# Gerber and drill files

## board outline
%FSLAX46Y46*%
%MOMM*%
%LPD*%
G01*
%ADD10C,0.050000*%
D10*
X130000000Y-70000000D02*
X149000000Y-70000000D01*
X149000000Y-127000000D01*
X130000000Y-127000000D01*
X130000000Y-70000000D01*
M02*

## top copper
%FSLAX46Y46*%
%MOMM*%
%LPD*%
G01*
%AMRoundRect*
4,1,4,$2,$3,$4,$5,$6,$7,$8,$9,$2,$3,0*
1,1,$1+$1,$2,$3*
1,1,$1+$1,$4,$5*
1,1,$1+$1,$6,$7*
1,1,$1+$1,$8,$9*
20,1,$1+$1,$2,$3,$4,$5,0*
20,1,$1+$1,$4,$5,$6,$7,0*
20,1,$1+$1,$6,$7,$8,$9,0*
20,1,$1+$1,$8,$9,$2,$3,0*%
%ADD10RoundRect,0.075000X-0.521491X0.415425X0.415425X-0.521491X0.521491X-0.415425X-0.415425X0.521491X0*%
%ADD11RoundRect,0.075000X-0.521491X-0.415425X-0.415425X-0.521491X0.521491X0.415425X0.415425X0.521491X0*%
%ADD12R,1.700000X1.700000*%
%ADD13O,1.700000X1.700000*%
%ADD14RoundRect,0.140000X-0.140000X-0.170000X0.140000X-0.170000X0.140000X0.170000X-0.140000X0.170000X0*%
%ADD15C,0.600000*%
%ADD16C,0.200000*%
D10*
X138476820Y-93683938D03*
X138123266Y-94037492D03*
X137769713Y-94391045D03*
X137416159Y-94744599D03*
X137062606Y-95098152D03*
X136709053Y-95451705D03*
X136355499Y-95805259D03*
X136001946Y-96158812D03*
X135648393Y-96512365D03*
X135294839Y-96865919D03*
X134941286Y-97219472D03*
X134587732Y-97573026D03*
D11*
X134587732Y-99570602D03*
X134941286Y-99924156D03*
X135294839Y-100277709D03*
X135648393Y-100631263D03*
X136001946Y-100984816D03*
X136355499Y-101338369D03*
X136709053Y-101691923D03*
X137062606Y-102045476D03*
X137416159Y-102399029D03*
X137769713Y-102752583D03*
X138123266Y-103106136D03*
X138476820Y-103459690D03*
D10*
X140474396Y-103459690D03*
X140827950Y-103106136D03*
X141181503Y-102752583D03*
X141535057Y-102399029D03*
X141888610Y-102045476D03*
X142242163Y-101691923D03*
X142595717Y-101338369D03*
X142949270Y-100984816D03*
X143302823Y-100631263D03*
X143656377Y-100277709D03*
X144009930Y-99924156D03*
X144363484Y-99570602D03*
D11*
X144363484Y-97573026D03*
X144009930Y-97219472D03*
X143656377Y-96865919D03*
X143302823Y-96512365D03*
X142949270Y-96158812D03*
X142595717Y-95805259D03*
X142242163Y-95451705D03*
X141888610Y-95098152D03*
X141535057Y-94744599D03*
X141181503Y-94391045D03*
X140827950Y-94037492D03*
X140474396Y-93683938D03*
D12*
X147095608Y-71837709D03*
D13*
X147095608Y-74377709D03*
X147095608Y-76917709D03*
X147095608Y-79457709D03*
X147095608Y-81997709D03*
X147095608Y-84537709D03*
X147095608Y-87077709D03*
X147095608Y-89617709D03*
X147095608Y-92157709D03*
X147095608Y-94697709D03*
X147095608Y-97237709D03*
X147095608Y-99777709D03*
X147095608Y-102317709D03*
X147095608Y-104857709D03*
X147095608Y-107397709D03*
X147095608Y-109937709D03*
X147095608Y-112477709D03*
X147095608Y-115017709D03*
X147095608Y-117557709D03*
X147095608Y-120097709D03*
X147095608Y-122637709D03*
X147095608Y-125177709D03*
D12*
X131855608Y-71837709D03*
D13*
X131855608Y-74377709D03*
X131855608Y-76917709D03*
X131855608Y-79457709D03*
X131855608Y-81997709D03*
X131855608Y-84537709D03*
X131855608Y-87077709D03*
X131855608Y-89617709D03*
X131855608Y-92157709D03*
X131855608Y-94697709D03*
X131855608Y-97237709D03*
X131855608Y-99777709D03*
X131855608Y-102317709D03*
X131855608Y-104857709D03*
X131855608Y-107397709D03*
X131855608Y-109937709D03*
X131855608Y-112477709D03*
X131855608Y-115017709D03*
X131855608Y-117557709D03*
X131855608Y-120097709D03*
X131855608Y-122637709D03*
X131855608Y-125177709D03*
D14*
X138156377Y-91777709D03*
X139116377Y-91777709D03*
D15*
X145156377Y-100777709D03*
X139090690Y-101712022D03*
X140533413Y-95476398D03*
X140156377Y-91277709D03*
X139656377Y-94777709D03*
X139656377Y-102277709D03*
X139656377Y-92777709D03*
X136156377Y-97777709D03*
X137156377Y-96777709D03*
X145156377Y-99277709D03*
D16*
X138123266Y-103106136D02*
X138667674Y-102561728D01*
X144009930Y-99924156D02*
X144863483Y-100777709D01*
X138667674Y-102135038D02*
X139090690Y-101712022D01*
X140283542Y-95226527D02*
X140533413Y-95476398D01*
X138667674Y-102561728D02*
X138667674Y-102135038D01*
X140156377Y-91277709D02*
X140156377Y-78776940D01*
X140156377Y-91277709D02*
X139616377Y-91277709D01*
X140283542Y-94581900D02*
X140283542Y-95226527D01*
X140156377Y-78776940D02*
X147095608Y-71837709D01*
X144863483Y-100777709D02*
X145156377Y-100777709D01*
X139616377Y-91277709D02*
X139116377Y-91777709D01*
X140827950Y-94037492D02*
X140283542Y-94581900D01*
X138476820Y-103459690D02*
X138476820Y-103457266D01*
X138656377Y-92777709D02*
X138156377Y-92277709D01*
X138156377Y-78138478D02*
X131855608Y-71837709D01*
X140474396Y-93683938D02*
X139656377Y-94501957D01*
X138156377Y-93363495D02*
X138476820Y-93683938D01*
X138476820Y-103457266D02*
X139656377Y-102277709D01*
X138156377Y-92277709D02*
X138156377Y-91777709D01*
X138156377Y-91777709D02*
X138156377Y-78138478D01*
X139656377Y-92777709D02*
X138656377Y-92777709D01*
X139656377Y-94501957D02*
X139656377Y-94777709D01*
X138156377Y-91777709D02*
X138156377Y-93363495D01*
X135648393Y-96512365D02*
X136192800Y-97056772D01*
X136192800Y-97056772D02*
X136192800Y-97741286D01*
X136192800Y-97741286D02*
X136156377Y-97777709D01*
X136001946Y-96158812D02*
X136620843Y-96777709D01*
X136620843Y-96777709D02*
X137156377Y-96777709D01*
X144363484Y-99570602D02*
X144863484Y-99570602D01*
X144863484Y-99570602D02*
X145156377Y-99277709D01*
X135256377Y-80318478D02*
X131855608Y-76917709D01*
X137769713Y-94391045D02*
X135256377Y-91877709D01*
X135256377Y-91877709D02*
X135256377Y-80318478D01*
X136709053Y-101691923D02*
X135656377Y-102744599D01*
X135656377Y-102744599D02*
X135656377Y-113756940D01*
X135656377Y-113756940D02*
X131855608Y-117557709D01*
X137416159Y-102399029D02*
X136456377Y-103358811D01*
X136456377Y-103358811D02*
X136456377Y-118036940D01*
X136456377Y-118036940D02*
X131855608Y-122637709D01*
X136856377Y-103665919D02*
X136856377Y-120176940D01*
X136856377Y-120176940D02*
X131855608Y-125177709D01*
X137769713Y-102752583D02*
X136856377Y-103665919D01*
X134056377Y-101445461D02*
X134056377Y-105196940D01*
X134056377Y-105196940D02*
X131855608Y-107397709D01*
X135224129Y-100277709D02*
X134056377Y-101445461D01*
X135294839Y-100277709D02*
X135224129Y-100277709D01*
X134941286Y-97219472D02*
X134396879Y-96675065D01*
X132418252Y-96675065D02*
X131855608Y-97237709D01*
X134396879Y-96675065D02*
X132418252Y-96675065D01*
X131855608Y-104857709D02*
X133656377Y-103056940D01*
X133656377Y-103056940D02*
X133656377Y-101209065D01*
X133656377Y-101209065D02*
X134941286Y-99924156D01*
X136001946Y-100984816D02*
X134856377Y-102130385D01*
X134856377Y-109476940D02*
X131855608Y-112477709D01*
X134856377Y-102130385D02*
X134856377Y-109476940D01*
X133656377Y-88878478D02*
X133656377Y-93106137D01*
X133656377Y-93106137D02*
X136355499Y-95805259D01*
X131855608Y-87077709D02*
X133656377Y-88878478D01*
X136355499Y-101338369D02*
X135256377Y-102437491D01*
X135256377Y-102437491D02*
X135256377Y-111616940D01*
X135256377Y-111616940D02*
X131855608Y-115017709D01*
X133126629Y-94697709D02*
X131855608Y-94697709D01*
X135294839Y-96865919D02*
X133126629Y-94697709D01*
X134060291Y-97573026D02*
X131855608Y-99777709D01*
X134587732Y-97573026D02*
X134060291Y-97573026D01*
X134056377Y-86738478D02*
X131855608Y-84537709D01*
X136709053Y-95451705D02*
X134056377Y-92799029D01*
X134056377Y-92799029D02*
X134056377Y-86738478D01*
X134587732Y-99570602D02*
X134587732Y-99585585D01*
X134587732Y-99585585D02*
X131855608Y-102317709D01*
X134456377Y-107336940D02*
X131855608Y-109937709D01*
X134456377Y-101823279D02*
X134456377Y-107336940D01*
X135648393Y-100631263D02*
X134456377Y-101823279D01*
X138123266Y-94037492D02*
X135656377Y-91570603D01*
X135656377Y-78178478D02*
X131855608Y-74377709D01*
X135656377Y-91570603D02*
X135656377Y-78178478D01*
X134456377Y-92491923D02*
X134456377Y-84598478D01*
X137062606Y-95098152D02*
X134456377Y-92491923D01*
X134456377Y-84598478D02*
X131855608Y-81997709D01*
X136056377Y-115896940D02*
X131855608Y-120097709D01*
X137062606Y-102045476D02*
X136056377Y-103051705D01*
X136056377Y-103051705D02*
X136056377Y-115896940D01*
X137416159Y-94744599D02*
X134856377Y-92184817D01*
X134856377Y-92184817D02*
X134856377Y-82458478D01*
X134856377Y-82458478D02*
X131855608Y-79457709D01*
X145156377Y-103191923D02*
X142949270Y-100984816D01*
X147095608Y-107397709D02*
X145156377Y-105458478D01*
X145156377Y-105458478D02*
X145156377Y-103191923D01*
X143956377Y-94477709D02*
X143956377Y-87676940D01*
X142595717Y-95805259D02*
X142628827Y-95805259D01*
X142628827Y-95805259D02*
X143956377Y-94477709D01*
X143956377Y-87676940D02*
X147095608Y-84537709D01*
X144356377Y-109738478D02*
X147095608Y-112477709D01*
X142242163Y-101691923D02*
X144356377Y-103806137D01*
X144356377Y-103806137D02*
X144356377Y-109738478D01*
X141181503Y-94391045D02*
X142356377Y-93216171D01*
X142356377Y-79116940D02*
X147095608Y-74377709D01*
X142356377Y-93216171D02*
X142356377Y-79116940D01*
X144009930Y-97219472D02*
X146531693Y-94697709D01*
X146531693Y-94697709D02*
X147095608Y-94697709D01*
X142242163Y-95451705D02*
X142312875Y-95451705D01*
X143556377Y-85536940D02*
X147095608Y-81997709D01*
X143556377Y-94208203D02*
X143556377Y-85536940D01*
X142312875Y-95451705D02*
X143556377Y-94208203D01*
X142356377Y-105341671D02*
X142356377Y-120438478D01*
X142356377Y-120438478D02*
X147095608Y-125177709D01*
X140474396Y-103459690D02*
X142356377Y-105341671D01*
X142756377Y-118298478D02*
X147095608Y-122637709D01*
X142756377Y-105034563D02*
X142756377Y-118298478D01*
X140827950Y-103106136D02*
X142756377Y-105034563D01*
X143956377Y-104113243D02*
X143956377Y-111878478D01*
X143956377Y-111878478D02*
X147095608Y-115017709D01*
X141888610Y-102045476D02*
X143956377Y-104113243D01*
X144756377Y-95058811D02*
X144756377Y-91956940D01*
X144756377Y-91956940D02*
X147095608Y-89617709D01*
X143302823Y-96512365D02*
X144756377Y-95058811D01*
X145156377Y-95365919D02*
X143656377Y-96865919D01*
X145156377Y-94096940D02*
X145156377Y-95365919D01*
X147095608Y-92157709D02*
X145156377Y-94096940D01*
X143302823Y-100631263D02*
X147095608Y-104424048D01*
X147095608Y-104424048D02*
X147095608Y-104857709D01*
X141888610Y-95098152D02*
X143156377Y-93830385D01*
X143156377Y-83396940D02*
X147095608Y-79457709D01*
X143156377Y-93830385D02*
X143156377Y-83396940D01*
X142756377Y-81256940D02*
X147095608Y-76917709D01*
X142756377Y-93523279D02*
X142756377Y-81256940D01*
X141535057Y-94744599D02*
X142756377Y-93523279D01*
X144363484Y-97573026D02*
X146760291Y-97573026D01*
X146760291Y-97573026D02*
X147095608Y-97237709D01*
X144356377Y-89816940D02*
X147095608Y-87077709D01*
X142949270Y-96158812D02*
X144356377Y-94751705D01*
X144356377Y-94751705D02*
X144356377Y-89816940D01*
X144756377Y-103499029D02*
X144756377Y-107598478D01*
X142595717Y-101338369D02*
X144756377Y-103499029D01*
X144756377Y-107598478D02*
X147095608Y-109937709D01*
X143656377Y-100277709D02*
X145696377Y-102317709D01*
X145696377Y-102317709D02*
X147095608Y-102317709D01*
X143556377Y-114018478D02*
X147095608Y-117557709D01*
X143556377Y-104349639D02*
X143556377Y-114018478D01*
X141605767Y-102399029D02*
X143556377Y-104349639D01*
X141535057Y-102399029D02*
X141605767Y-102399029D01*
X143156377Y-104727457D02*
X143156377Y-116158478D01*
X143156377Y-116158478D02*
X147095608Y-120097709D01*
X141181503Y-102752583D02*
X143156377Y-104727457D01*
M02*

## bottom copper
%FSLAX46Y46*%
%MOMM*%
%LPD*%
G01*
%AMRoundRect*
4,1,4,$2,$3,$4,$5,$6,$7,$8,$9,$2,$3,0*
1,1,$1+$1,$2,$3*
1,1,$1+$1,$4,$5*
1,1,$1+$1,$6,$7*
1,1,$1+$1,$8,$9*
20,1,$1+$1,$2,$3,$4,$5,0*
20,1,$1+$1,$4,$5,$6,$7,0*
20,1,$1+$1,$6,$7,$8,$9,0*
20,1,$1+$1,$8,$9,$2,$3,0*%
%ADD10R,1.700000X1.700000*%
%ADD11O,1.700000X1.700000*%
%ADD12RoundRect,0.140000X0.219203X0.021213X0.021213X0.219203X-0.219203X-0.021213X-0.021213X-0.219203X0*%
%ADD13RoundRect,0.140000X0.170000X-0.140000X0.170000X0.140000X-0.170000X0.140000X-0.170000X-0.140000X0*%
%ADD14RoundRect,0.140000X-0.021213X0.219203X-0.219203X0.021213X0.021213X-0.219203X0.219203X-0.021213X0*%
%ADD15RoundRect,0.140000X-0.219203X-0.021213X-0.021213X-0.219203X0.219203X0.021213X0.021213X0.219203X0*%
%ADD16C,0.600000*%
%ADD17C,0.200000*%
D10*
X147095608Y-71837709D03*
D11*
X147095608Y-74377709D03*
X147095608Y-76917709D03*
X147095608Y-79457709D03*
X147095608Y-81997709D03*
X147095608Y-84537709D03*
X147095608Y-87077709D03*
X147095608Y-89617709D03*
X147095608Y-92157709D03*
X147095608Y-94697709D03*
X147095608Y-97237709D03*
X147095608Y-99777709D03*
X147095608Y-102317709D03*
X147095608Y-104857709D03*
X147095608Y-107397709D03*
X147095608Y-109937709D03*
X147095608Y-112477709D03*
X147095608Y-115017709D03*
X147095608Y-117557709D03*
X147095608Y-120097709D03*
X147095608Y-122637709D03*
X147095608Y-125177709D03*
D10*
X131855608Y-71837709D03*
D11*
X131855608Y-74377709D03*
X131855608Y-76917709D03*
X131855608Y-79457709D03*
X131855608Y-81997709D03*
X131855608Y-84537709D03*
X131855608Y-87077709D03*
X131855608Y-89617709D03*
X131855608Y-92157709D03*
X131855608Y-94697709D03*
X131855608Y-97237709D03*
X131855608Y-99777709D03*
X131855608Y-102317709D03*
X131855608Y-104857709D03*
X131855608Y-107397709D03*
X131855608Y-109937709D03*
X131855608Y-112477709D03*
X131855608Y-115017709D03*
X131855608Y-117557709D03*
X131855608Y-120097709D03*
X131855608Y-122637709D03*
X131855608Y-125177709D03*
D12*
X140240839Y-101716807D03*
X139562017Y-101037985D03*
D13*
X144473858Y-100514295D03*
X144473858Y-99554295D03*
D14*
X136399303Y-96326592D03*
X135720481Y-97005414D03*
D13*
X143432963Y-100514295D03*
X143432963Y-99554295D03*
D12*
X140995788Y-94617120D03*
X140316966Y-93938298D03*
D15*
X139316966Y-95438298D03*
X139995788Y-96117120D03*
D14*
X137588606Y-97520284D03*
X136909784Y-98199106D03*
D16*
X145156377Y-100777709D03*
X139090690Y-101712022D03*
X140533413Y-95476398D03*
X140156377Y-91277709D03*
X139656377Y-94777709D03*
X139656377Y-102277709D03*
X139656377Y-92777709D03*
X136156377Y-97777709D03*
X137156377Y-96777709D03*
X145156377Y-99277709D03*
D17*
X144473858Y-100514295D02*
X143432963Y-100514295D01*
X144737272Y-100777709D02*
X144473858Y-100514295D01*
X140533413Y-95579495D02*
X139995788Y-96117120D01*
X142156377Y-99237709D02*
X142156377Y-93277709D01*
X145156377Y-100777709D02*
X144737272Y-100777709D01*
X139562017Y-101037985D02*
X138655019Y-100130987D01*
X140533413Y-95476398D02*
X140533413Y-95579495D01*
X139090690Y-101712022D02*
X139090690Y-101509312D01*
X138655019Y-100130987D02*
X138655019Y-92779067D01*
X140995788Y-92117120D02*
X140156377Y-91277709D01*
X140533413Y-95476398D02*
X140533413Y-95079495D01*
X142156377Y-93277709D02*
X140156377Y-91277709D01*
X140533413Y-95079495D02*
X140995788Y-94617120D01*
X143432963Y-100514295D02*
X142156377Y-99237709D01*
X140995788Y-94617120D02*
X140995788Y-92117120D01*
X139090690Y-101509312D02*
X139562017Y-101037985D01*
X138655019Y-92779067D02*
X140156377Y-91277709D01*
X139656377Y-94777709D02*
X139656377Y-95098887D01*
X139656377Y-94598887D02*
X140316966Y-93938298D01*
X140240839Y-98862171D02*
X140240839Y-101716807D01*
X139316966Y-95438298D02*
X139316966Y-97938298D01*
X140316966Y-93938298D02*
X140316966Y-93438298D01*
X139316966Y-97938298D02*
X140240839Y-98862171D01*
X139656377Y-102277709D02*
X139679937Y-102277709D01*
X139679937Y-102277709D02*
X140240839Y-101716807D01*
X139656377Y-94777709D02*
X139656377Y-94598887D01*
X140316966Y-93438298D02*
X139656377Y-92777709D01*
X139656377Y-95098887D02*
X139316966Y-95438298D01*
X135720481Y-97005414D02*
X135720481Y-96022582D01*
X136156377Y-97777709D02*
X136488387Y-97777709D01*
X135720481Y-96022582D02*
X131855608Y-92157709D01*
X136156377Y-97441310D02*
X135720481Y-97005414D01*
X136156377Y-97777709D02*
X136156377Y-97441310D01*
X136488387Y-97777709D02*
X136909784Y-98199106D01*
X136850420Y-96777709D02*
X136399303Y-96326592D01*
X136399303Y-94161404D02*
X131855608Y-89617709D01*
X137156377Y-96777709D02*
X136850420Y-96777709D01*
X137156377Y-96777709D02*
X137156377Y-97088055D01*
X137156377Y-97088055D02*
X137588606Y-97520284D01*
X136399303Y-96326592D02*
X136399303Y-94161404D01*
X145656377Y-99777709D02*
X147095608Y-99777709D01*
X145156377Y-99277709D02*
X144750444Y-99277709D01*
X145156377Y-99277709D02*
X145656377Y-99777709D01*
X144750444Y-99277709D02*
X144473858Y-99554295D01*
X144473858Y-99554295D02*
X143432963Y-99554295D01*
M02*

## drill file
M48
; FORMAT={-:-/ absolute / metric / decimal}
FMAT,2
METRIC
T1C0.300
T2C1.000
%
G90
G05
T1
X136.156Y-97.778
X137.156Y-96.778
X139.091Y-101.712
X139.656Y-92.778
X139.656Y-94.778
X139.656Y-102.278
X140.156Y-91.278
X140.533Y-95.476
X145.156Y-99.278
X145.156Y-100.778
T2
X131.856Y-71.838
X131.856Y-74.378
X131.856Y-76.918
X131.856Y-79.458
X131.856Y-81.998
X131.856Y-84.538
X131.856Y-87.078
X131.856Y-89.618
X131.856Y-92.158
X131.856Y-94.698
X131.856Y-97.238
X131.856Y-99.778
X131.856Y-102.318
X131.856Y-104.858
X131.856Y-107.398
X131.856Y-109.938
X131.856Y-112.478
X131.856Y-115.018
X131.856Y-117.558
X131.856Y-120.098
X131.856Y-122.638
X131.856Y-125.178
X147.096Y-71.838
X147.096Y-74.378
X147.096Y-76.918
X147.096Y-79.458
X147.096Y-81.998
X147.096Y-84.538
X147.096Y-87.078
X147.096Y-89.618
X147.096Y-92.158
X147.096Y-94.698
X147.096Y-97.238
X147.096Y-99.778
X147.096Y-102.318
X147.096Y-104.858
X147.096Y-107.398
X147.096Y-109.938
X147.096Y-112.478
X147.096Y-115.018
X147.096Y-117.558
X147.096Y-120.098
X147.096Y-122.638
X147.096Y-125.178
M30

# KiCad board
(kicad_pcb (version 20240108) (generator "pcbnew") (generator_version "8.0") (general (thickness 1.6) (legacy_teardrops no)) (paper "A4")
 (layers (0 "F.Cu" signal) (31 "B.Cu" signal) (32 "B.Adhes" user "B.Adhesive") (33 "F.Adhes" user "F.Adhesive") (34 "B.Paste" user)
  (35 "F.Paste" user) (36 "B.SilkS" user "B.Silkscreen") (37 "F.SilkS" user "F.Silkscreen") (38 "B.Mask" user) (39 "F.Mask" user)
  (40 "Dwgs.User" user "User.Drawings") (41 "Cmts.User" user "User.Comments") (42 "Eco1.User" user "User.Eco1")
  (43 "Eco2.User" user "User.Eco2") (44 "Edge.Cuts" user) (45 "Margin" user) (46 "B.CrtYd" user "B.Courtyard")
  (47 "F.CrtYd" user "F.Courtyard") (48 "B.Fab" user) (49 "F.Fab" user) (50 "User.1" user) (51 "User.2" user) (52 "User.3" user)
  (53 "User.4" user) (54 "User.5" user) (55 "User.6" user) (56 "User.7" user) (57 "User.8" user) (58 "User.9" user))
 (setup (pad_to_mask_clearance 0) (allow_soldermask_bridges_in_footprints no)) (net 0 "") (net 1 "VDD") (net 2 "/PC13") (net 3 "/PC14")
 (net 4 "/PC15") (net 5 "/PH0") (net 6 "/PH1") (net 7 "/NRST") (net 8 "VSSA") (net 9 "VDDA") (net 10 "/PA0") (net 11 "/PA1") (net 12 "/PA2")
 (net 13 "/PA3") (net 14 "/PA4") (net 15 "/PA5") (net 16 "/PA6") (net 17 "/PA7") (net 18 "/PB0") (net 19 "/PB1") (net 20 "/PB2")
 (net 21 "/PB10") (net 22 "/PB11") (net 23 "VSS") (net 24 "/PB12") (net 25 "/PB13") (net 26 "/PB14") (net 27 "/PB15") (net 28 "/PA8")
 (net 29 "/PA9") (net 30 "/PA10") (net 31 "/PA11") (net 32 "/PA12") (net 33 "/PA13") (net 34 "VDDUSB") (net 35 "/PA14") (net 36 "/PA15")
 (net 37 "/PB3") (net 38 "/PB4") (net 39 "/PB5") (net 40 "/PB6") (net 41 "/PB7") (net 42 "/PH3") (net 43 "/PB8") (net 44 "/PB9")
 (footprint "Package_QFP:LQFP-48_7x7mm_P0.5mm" (layer "F.Cu") (at 139.475608 98.571814 -45)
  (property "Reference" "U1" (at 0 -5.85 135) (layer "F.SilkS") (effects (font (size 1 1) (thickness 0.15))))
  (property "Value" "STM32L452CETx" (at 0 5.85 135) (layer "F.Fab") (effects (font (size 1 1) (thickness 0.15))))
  (pad "1" smd roundrect (at -4.1625 -2.75 315) (size 1.475 0.3) (layers "F.Cu" "F.Paste" "F.Mask") (roundrect_rratio 0.25) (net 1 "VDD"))
  (pad "2" smd roundrect (at -4.1625 -2.25 315) (size 1.475 0.3) (layers "F.Cu" "F.Paste" "F.Mask") (roundrect_rratio 0.25) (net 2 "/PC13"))
  (pad "3" smd roundrect (at -4.1625 -1.75 315) (size 1.475 0.3) (layers "F.Cu" "F.Paste" "F.Mask") (roundrect_rratio 0.25) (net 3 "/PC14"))
  (pad "4" smd roundrect (at -4.1625 -1.249999 315) (size 1.475 0.3) (layers "F.Cu" "F.Paste" "F.Mask") (roundrect_rratio 0.25)
   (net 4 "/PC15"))
  (pad "5" smd roundrect (at -4.1625 -0.75 315) (size 1.475 0.3) (layers "F.Cu" "F.Paste" "F.Mask") (roundrect_rratio 0.25) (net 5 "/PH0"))
  (pad "6" smd roundrect (at -4.1625 -0.25 315) (size 1.475 0.3) (layers "F.Cu" "F.Paste" "F.Mask") (roundrect_rratio 0.25) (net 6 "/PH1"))
  (pad "7" smd roundrect (at -4.1625 0.25 315) (size 1.475 0.3) (layers "F.Cu" "F.Paste" "F.Mask") (roundrect_rratio 0.25) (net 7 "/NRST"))
  (pad "8" smd roundrect (at -4.1625 0.75 315) (size 1.475 0.3) (layers "F.Cu" "F.Paste" "F.Mask") (roundrect_rratio 0.25) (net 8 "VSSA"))
  (pad "9" smd roundrect (at -4.1625 1.249999 315) (size 1.475 0.3) (layers "F.Cu" "F.Paste" "F.Mask") (roundrect_rratio 0.25)
   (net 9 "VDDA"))
  (pad "10" smd roundrect (at -4.1625 1.75 315) (size 1.475 0.3) (layers "F.Cu" "F.Paste" "F.Mask") (roundrect_rratio 0.25) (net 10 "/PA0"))
  (pad "11" smd roundrect (at -4.1625 2.25 315) (size 1.475 0.3) (layers "F.Cu" "F.Paste" "F.Mask") (roundrect_rratio 0.25) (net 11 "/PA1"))
  (pad "12" smd roundrect (at -4.1625 2.75 315) (size 1.475 0.3) (layers "F.Cu" "F.Paste" "F.Mask") (roundrect_rratio 0.25) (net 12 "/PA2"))
  (pad "13" smd roundrect (at -2.75 4.1625 315) (size 0.3 1.475) (layers "F.Cu" "F.Paste" "F.Mask") (roundrect_rratio 0.25) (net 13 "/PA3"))
  (pad "14" smd roundrect (at -2.25 4.1625 315) (size 0.3 1.475) (layers "F.Cu" "F.Paste" "F.Mask") (roundrect_rratio 0.25) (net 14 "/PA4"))
  (pad "15" smd roundrect (at -1.75 4.1625 315) (size 0.3 1.475) (layers "F.Cu" "F.Paste" "F.Mask") (roundrect_rratio 0.25) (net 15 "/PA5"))
  (pad "16" smd roundrect (at -1.249999 4.1625 315) (size 0.3 1.475) (layers "F.Cu" "F.Paste" "F.Mask") (roundrect_rratio 0.25)
   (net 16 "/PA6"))
  (pad "17" smd roundrect (at -0.75 4.1625 315) (size 0.3 1.475) (layers "F.Cu" "F.Paste" "F.Mask") (roundrect_rratio 0.25) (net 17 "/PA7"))
  (pad "18" smd roundrect (at -0.25 4.1625 315) (size 0.3 1.475) (layers "F.Cu" "F.Paste" "F.Mask") (roundrect_rratio 0.25) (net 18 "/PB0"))
  (pad "19" smd roundrect (at 0.25 4.1625 315) (size 0.3 1.475) (layers "F.Cu" "F.Paste" "F.Mask") (roundrect_rratio 0.25) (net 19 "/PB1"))
  (pad "20" smd roundrect (at 0.75 4.1625 315) (size 0.3 1.475) (layers "F.Cu" "F.Paste" "F.Mask") (roundrect_rratio 0.25) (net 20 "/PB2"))
  (pad "21" smd roundrect (at 1.249999 4.1625 315) (size 0.3 1.475) (layers "F.Cu" "F.Paste" "F.Mask") (roundrect_rratio 0.25)
   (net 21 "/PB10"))
  (pad "22" smd roundrect (at 1.75 4.1625 315) (size 0.3 1.475) (layers "F.Cu" "F.Paste" "F.Mask") (roundrect_rratio 0.25) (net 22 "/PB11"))
  (pad "23" smd roundrect (at 2.25 4.1625 315) (size 0.3 1.475) (layers "F.Cu" "F.Paste" "F.Mask") (roundrect_rratio 0.25) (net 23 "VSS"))
  (pad "24" smd roundrect (at 2.75 4.1625 315) (size 0.3 1.475) (layers "F.Cu" "F.Paste" "F.Mask") (roundrect_rratio 0.25) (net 1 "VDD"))
  (pad "25" smd roundrect (at 4.1625 2.75 315) (size 1.475 0.3) (layers "F.Cu" "F.Paste" "F.Mask") (roundrect_rratio 0.25) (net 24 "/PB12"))
  (pad "26" smd roundrect (at 4.1625 2.25 315) (size 1.475 0.3) (layers "F.Cu" "F.Paste" "F.Mask") (roundrect_rratio 0.25) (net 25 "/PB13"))
  (pad "27" smd roundrect (at 4.1625 1.75 315) (size 1.475 0.3) (layers "F.Cu" "F.Paste" "F.Mask") (roundrect_rratio 0.25) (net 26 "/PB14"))
  (pad "28" smd roundrect (at 4.1625 1.249999 315) (size 1.475 0.3) (layers "F.Cu" "F.Paste" "F.Mask") (roundrect_rratio 0.25)
   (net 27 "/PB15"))
  (pad "29" smd roundrect (at 4.1625 0.75 315) (size 1.475 0.3) (layers "F.Cu" "F.Paste" "F.Mask") (roundrect_rratio 0.25) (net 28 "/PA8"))
  (pad "30" smd roundrect (at 4.1625 0.25 315) (size 1.475 0.3) (layers "F.Cu" "F.Paste" "F.Mask") (roundrect_rratio 0.25) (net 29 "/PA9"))
  (pad "31" smd roundrect (at 4.1625 -0.25 315) (size 1.475 0.3) (layers "F.Cu" "F.Paste" "F.Mask") (roundrect_rratio 0.25) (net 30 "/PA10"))
  (pad "32" smd roundrect (at 4.1625 -0.75 315) (size 1.475 0.3) (layers "F.Cu" "F.Paste" "F.Mask") (roundrect_rratio 0.25) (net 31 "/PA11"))
  (pad "33" smd roundrect (at 4.1625 -1.249999 315) (size 1.475 0.3) (layers "F.Cu" "F.Paste" "F.Mask") (roundrect_rratio 0.25)
   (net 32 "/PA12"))
  (pad "34" smd roundrect (at 4.1625 -1.75 315) (size 1.475 0.3) (layers "F.Cu" "F.Paste" "F.Mask") (roundrect_rratio 0.25) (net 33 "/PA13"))
  (pad "35" smd roundrect (at 4.1625 -2.25 315) (size 1.475 0.3) (layers "F.Cu" "F.Paste" "F.Mask") (roundrect_rratio 0.25) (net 23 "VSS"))
  (pad "36" smd roundrect (at 4.1625 -2.75 315) (size 1.475 0.3) (layers "F.Cu" "F.Paste" "F.Mask") (roundrect_rratio 0.25)
   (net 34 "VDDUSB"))
  (pad "37" smd roundrect (at 2.75 -4.1625 315) (size 0.3 1.475) (layers "F.Cu" "F.Paste" "F.Mask") (roundrect_rratio 0.25) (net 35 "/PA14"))
  (pad "38" smd roundrect (at 2.25 -4.1625 315) (size 0.3 1.475) (layers "F.Cu" "F.Paste" "F.Mask") (roundrect_rratio 0.25) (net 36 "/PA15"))
  (pad "39" smd roundrect (at 1.75 -4.1625 315) (size 0.3 1.475) (layers "F.Cu" "F.Paste" "F.Mask") (roundrect_rratio 0.25) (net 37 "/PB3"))
  (pad "40" smd roundrect (at 1.249999 -4.1625 315) (size 0.3 1.475) (layers "F.Cu" "F.Paste" "F.Mask") (roundrect_rratio 0.25)
   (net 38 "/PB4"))
  (pad "41" smd roundrect (at 0.75 -4.1625 315) (size 0.3 1.475) (layers "F.Cu" "F.Paste" "F.Mask") (roundrect_rratio 0.25) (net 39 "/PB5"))
  (pad "42" smd roundrect (at 0.25 -4.1625 315) (size 0.3 1.475) (layers "F.Cu" "F.Paste" "F.Mask") (roundrect_rratio 0.25) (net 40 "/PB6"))
  (pad "43" smd roundrect (at -0.25 -4.1625 315) (size 0.3 1.475) (layers "F.Cu" "F.Paste" "F.Mask") (roundrect_rratio 0.25) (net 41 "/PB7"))
  (pad "44" smd roundrect (at -0.75 -4.1625 315) (size 0.3 1.475) (layers "F.Cu" "F.Paste" "F.Mask") (roundrect_rratio 0.25) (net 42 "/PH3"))
  (pad "45" smd roundrect (at -1.249999 -4.1625 315) (size 0.3 1.475) (layers "F.Cu" "F.Paste" "F.Mask") (roundrect_rratio 0.25)
   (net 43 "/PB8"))
  (pad "46" smd roundrect (at -1.75 -4.1625 315) (size 0.3 1.475) (layers "F.Cu" "F.Paste" "F.Mask") (roundrect_rratio 0.25) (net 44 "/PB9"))
  (pad "47" smd roundrect (at -2.25 -4.1625 315) (size 0.3 1.475) (layers "F.Cu" "F.Paste" "F.Mask") (roundrect_rratio 0.25) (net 23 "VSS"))
  (pad "48" smd roundrect (at -2.75 -4.1625 315) (size 0.3 1.475) (layers "F.Cu" "F.Paste" "F.Mask") (roundrect_rratio 0.25) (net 1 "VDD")))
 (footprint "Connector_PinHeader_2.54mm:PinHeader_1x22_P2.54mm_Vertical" (layer "F.Cu") (at 147.095608 71.837709)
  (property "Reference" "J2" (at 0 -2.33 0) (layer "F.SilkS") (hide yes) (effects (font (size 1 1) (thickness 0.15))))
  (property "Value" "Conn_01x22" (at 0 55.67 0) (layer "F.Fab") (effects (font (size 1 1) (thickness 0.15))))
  (pad "1" thru_hole rect (at 0 0) (size 1.7 1.7) (drill 1) (layers "*.Cu" "*.Mask") (remove_unused_layers no) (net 23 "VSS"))
  (pad "2" thru_hole oval (at 0 2.54) (size 1.7 1.7) (drill 1) (layers "*.Cu" "*.Mask") (remove_unused_layers no) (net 44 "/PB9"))
  (pad "3" thru_hole oval (at 0 5.08) (size 1.7 1.7) (drill 1) (layers "*.Cu" "*.Mask") (remove_unused_layers no) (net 43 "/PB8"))
  (pad "4" thru_hole oval (at 0 7.62) (size 1.7 1.7) (drill 1) (layers "*.Cu" "*.Mask") (remove_unused_layers no) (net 42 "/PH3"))
  (pad "5" thru_hole oval (at 0 10.16) (size 1.7 1.7) (drill 1) (layers "*.Cu" "*.Mask") (remove_unused_layers no) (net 41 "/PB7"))
  (pad "6" thru_hole oval (at 0 12.7) (size 1.7 1.7) (drill 1) (layers "*.Cu" "*.Mask") (remove_unused_layers no) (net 40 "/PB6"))
  (pad "7" thru_hole oval (at 0 15.24) (size 1.7 1.7) (drill 1) (layers "*.Cu" "*.Mask") (remove_unused_layers no) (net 39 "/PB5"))
  (pad "8" thru_hole oval (at 0 17.78) (size 1.7 1.7) (drill 1) (layers "*.Cu" "*.Mask") (remove_unused_layers no) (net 38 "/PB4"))
  (pad "9" thru_hole oval (at 0 20.32) (size 1.7 1.7) (drill 1) (layers "*.Cu" "*.Mask") (remove_unused_layers no) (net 37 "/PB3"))
  (pad "10" thru_hole oval (at 0 22.86) (size 1.7 1.7) (drill 1) (layers "*.Cu" "*.Mask") (remove_unused_layers no) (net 36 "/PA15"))
  (pad "11" thru_hole oval (at 0 25.4) (size 1.7 1.7) (drill 1) (layers "*.Cu" "*.Mask") (remove_unused_layers no) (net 35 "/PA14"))
  (pad "12" thru_hole oval (at 0 27.94) (size 1.7 1.7) (drill 1) (layers "*.Cu" "*.Mask") (remove_unused_layers no) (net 34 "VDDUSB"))
  (pad "13" thru_hole oval (at 0 30.48) (size 1.7 1.7) (drill 1) (layers "*.Cu" "*.Mask") (remove_unused_layers no) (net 33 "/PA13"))
  (pad "14" thru_hole oval (at 0 33.02) (size 1.7 1.7) (drill 1) (layers "*.Cu" "*.Mask") (remove_unused_layers no) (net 32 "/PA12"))
  (pad "15" thru_hole oval (at 0 35.56) (size 1.7 1.7) (drill 1) (layers "*.Cu" "*.Mask") (remove_unused_layers no) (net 31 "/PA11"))
  (pad "16" thru_hole oval (at 0 38.1) (size 1.7 1.7) (drill 1) (layers "*.Cu" "*.Mask") (remove_unused_layers no) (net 30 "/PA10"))
  (pad "17" thru_hole oval (at 0 40.64) (size 1.7 1.7) (drill 1) (layers "*.Cu" "*.Mask") (remove_unused_layers no) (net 29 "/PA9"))
  (pad "18" thru_hole oval (at 0 43.18) (size 1.7 1.7) (drill 1) (layers "*.Cu" "*.Mask") (remove_unused_layers no) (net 28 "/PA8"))
  (pad "19" thru_hole oval (at 0 45.72) (size 1.7 1.7) (drill 1) (layers "*.Cu" "*.Mask") (remove_unused_layers no) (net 27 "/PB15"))
  (pad "20" thru_hole oval (at 0 48.26) (size 1.7 1.7) (drill 1) (layers "*.Cu" "*.Mask") (remove_unused_layers no) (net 26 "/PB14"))
  (pad "21" thru_hole oval (at 0 50.8) (size 1.7 1.7) (drill 1) (layers "*.Cu" "*.Mask") (remove_unused_layers no) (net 25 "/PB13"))
  (pad "22" thru_hole oval (at 0 53.34) (size 1.7 1.7) (drill 1) (layers "*.Cu" "*.Mask") (remove_unused_layers no) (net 24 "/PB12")))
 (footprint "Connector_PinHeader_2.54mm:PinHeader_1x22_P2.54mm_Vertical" (layer "F.Cu") (at 131.855608 71.837709)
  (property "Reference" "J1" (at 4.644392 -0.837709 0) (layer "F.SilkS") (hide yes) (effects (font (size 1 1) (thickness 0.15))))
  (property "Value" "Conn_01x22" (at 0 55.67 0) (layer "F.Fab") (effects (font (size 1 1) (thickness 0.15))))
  (pad "1" thru_hole rect (at 0 0) (size 1.7 1.7) (drill 1) (layers "*.Cu" "*.Mask") (remove_unused_layers no) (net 1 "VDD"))
  (pad "2" thru_hole oval (at 0 2.54) (size 1.7 1.7) (drill 1) (layers "*.Cu" "*.Mask") (remove_unused_layers no) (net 2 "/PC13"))
  (pad "3" thru_hole oval (at 0 5.08) (size 1.7 1.7) (drill 1) (layers "*.Cu" "*.Mask") (remove_unused_layers no) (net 3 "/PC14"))
  (pad "4" thru_hole oval (at 0 7.62) (size 1.7 1.7) (drill 1) (layers "*.Cu" "*.Mask") (remove_unused_layers no) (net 4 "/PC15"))
  (pad "5" thru_hole oval (at 0 10.16) (size 1.7 1.7) (drill 1) (layers "*.Cu" "*.Mask") (remove_unused_layers no) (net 5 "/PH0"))
  (pad "6" thru_hole oval (at 0 12.7) (size 1.7 1.7) (drill 1) (layers "*.Cu" "*.Mask") (remove_unused_layers no) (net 6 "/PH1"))
  (pad "7" thru_hole oval (at 0 15.24) (size 1.7 1.7) (drill 1) (layers "*.Cu" "*.Mask") (remove_unused_layers no) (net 7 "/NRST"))
  (pad "8" thru_hole oval (at 0 17.78) (size 1.7 1.7) (drill 1) (layers "*.Cu" "*.Mask") (remove_unused_layers no) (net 8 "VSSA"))
  (pad "9" thru_hole oval (at 0 20.32) (size 1.7 1.7) (drill 1) (layers "*.Cu" "*.Mask") (remove_unused_layers no) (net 9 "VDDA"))
  (pad "10" thru_hole oval (at 0 22.86) (size 1.7 1.7) (drill 1) (layers "*.Cu" "*.Mask") (remove_unused_layers no) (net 10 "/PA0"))
  (pad "11" thru_hole oval (at 0 25.4) (size 1.7 1.7) (drill 1) (layers "*.Cu" "*.Mask") (remove_unused_layers no) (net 11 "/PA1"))
  (pad "12" thru_hole oval (at 0 27.94) (size 1.7 1.7) (drill 1) (layers "*.Cu" "*.Mask") (remove_unused_layers no) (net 12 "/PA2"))
  (pad "13" thru_hole oval (at 0 30.48) (size 1.7 1.7) (drill 1) (layers "*.Cu" "*.Mask") (remove_unused_layers no) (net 13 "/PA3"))
  (pad "14" thru_hole oval (at 0 33.02) (size 1.7 1.7) (drill 1) (layers "*.Cu" "*.Mask") (remove_unused_layers no) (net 14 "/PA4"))
  (pad "15" thru_hole oval (at 0 35.56) (size 1.7 1.7) (drill 1) (layers "*.Cu" "*.Mask") (remove_unused_layers no) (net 15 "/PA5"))
  (pad "16" thru_hole oval (at 0 38.1) (size 1.7 1.7) (drill 1) (layers "*.Cu" "*.Mask") (remove_unused_layers no) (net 16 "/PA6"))
  (pad "17" thru_hole oval (at 0 40.64) (size 1.7 1.7) (drill 1) (layers "*.Cu" "*.Mask") (remove_unused_layers no) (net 17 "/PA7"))
  (pad "18" thru_hole oval (at 0 43.18) (size 1.7 1.7) (drill 1) (layers "*.Cu" "*.Mask") (remove_unused_layers no) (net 18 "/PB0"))
  (pad "19" thru_hole oval (at 0 45.72) (size 1.7 1.7) (drill 1) (layers "*.Cu" "*.Mask") (remove_unused_layers no) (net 19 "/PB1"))
  (pad "20" thru_hole oval (at 0 48.26) (size 1.7 1.7) (drill 1) (layers "*.Cu" "*.Mask") (remove_unused_layers no) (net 20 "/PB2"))
  (pad "21" thru_hole oval (at 0 50.8) (size 1.7 1.7) (drill 1) (layers "*.Cu" "*.Mask") (remove_unused_layers no) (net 21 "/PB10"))
  (pad "22" thru_hole oval (at 0 53.34) (size 1.7 1.7) (drill 1) (layers "*.Cu" "*.Mask") (remove_unused_layers no) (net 22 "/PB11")))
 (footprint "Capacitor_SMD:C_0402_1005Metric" (layer "F.Cu") (at 138.636377 91.777709)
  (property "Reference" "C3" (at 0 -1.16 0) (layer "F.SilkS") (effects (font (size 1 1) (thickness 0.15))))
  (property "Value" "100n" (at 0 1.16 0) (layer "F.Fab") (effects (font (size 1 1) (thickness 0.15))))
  (pad "1" smd roundrect (at -0.48 0) (size 0.56 0.62) (layers "F.Cu" "F.Paste" "F.Mask") (roundrect_rratio 0.25) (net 1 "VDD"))
  (pad "2" smd roundrect (at 0.48 0) (size 0.56 0.62) (layers "F.Cu" "F.Paste" "F.Mask") (roundrect_rratio 0.25) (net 23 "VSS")))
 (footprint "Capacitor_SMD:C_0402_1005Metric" (layer "B.Cu") (at 139.901428 101.377396 135)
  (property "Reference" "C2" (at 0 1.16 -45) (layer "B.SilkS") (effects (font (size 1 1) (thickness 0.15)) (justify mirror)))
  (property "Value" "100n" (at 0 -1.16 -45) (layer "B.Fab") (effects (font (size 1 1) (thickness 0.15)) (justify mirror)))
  (pad "1" smd roundrect (at -0.48 0 135) (size 0.56 0.62) (layers "B.Cu" "B.Paste" "B.Mask") (roundrect_rratio 0.25) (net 1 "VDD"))
  (pad "2" smd roundrect (at 0.48 0 135) (size 0.56 0.62) (layers "B.Cu" "B.Paste" "B.Mask") (roundrect_rratio 0.25) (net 23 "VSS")))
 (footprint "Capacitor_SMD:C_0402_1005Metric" (layer "B.Cu") (at 144.473858 100.034295 90)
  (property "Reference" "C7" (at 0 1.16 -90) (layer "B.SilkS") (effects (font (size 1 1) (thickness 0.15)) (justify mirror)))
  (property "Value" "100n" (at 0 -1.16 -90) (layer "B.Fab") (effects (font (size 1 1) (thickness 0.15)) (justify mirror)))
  (pad "1" smd roundrect (at -0.48 0 90) (size 0.56 0.62) (layers "B.Cu" "B.Paste" "B.Mask") (roundrect_rratio 0.25) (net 23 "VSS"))
  (pad "2" smd roundrect (at 0.48 0 90) (size 0.56 0.62) (layers "B.Cu" "B.Paste" "B.Mask") (roundrect_rratio 0.25) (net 34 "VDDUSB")))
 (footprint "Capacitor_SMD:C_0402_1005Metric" (layer "B.Cu") (at 136.059892 96.666003 -135)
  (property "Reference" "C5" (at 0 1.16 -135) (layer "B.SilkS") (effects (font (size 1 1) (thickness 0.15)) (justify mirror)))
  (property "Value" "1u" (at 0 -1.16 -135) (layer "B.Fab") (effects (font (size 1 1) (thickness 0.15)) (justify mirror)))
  (pad "1" smd roundrect (at -0.48 0 225) (size 0.56 0.62) (layers "B.Cu" "B.Paste" "B.Mask") (roundrect_rratio 0.25) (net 8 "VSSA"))
  (pad "2" smd roundrect (at 0.48 0 225) (size 0.56 0.62) (layers "B.Cu" "B.Paste" "B.Mask") (roundrect_rratio 0.25) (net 9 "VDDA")))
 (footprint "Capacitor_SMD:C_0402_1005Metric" (layer "B.Cu") (at 143.432963 100.034295 90)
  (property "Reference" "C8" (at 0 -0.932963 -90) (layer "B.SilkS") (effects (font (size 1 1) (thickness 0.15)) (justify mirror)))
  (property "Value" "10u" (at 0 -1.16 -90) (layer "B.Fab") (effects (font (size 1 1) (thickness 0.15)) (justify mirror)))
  (pad "1" smd roundrect (at -0.48 0 90) (size 0.56 0.62) (layers "B.Cu" "B.Paste" "B.Mask") (roundrect_rratio 0.25) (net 23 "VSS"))
  (pad "2" smd roundrect (at 0.48 0 90) (size 0.56 0.62) (layers "B.Cu" "B.Paste" "B.Mask") (roundrect_rratio 0.25) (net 34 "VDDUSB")))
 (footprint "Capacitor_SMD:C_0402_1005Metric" (layer "B.Cu") (at 140.656377 94.277709 135)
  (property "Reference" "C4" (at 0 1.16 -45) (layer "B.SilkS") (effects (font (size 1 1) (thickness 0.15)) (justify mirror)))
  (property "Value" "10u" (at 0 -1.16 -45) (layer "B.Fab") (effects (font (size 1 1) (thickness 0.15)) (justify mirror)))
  (pad "1" smd roundrect (at -0.48 0 135) (size 0.56 0.62) (layers "B.Cu" "B.Paste" "B.Mask") (roundrect_rratio 0.25) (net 23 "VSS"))
  (pad "2" smd roundrect (at 0.48 0 135) (size 0.56 0.62) (layers "B.Cu" "B.Paste" "B.Mask") (roundrect_rratio 0.25) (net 1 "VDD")))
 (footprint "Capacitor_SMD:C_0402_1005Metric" (layer "B.Cu") (at 139.656377 95.777709 -45)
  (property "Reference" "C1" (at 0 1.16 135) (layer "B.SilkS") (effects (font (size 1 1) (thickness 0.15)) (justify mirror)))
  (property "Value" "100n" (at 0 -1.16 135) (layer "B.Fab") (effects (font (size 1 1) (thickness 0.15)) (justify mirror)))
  (pad "1" smd roundrect (at -0.48 0 315) (size 0.56 0.62) (layers "B.Cu" "B.Paste" "B.Mask") (roundrect_rratio 0.25) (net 1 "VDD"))
  (pad "2" smd roundrect (at 0.48 0 315) (size 0.56 0.62) (layers "B.Cu" "B.Paste" "B.Mask") (roundrect_rratio 0.25) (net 23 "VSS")))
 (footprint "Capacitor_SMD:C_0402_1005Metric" (layer "B.Cu") (at 137.249195 97.859695 -135)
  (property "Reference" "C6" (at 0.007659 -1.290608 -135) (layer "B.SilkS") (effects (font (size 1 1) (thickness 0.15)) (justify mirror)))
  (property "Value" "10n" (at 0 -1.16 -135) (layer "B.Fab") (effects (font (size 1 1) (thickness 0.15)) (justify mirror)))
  (pad "1" smd roundrect (at -0.48 0 225) (size 0.56 0.62) (layers "B.Cu" "B.Paste" "B.Mask") (roundrect_rratio 0.25) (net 8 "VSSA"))
  (pad "2" smd roundrect (at 0.48 0 225) (size 0.56 0.62) (layers "B.Cu" "B.Paste" "B.Mask") (roundrect_rratio 0.25) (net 9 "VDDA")))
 (gr_rect (start 130 70) (end 149 127) (stroke (width 0.05) (type default)) (fill none) (layer "Edge.Cuts"))
 (segment (start 138.123266 103.106136) (end 138.667674 102.561728) (width 0.2) (layer "F.Cu") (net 23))
 (segment (start 144.00993 99.924156) (end 144.863483 100.777709) (width 0.2) (layer "F.Cu") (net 23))
 (segment (start 138.667674 102.135038) (end 139.09069 101.712022) (width 0.2) (layer "F.Cu") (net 23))
 (segment (start 140.283542 95.226527) (end 140.533413 95.476398) (width 0.2) (layer "F.Cu") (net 23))
 (segment (start 138.667674 102.561728) (end 138.667674 102.135038) (width 0.2) (layer "F.Cu") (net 23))
 (segment (start 140.156377 91.277709) (end 140.156377 78.77694) (width 0.2) (layer "F.Cu") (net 23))
 (segment (start 140.156377 91.277709) (end 139.616377 91.277709) (width 0.2) (layer "F.Cu") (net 23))
 (segment (start 140.283542 94.5819) (end 140.283542 95.226527) (width 0.2) (layer "F.Cu") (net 23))
 (segment (start 140.156377 78.77694) (end 147.095608 71.837709) (width 0.2) (layer "F.Cu") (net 23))
 (segment (start 144.863483 100.777709) (end 145.156377 100.777709) (width 0.2) (layer "F.Cu") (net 23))
 (segment (start 139.616377 91.277709) (end 139.116377 91.777709) (width 0.2) (layer "F.Cu") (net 23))
 (segment (start 140.82795 94.037492) (end 140.283542 94.5819) (width 0.2) (layer "F.Cu") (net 23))
 (via (at 145.156377 100.777709) (size 0.6) (drill 0.3) (layers "F.Cu" "B.Cu") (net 23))
 (via (at 139.09069 101.712022) (size 0.6) (drill 0.3) (layers "F.Cu" "B.Cu") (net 23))
 (via (at 140.533413 95.476398) (size 0.6) (drill 0.3) (layers "F.Cu" "B.Cu") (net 23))
 (via (at 140.156377 91.277709) (size 0.6) (drill 0.3) (layers "F.Cu" "B.Cu") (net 23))
 (segment (start 144.473858 100.514295) (end 143.432963 100.514295) (width 0.2) (layer "B.Cu") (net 23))
 (segment (start 144.737272 100.777709) (end 144.473858 100.514295) (width 0.2) (layer "B.Cu") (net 23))
 (segment (start 140.533413 95.579495) (end 139.995788 96.11712) (width 0.2) (layer "B.Cu") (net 23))
 (segment (start 142.156377 99.237709) (end 142.156377 93.277709) (width 0.2) (layer "B.Cu") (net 23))
 (segment (start 145.156377 100.777709) (end 144.737272 100.777709) (width 0.2) (layer "B.Cu") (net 23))
 (segment (start 139.562017 101.037985) (end 138.655019 100.130987) (width 0.2) (layer "B.Cu") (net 23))
 (segment (start 140.533413 95.476398) (end 140.533413 95.579495) (width 0.2) (layer "B.Cu") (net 23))
 (segment (start 139.09069 101.712022) (end 139.09069 101.509312) (width 0.2) (layer "B.Cu") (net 23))
 (segment (start 138.655019 100.130987) (end 138.655019 92.779067) (width 0.2) (layer "B.Cu") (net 23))
 (segment (start 140.995788 92.11712) (end 140.156377 91.277709) (width 0.2) (layer "B.Cu") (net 23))
 (segment (start 140.533413 95.476398) (end 140.533413 95.079495) (width 0.2) (layer "B.Cu") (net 23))
 (segment (start 142.156377 93.277709) (end 140.156377 91.277709) (width 0.2) (layer "B.Cu") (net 23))
 (segment (start 140.533413 95.079495) (end 140.995788 94.61712) (width 0.2) (layer "B.Cu") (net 23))
 (segment (start 143.432963 100.514295) (end 142.156377 99.237709) (width 0.2) (layer "B.Cu") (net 23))
 (segment (start 140.995788 94.61712) (end 140.995788 92.11712) (width 0.2) (layer "B.Cu") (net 23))
 (segment (start 139.09069 101.509312) (end 139.562017 101.037985) (width 0.2) (layer "B.Cu") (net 23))
 (segment (start 138.655019 92.779067) (end 140.156377 91.277709) (width 0.2) (layer "B.Cu") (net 23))
 (segment (start 138.47682 103.45969) (end 138.47682 103.457266) (width 0.2) (layer "F.Cu") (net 1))
 (segment (start 138.656377 92.777709) (end 138.156377 92.277709) (width 0.2) (layer "F.Cu") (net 1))
 (segment (start 138.156377 78.138478) (end 131.855608 71.837709) (width 0.2) (layer "F.Cu") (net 1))
 (segment (start 140.474396 93.683938) (end 139.656377 94.501957) (width 0.2) (layer "F.Cu") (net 1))
 (segment (start 138.156377 93.363495) (end 138.47682 93.683938) (width 0.2) (layer "F.Cu") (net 1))
 (segment (start 138.47682 103.457266) (end 139.656377 102.277709) (width 0.2) (layer "F.Cu") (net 1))
 (segment (start 138.156377 92.277709) (end 138.156377 91.777709) (width 0.2) (layer "F.Cu") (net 1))
 (segment (start 138.156377 91.777709) (end 138.156377 78.138478) (width 0.2) (layer "F.Cu") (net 1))
 (segment (start 139.656377 92.777709) (end 138.656377 92.777709) (width 0.2) (layer "F.Cu") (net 1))
 (segment (start 139.656377 94.501957) (end 139.656377 94.777709) (width 0.2) (layer "F.Cu") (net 1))
 (segment (start 138.156377 91.777709) (end 138.156377 93.363495) (width 0.2) (layer "F.Cu") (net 1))
 (via (at 139.656377 94.777709) (size 0.6) (drill 0.3) (layers "F.Cu" "B.Cu") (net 1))
 (via (at 139.656377 102.277709) (size 0.6) (drill 0.3) (layers "F.Cu" "B.Cu") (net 1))
 (via (at 139.656377 92.777709) (size 0.6) (drill 0.3) (layers "F.Cu" "B.Cu") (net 1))
 (segment (start 139.656377 94.777709) (end 139.656377 95.098887) (width 0.2) (layer "B.Cu") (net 1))
 (segment (start 139.656377 94.598887) (end 140.316966 93.938298) (width 0.2) (layer "B.Cu") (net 1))
 (segment (start 140.240839 98.862171) (end 140.240839 101.716807) (width 0.2) (layer "B.Cu") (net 1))
 (segment (start 139.316966 95.438298) (end 139.316966 97.938298) (width 0.2) (layer "B.Cu") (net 1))
 (segment (start 140.316966 93.938298) (end 140.316966 93.438298) (width 0.2) (layer "B.Cu") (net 1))
 (segment (start 139.316966 97.938298) (end 140.240839 98.862171) (width 0.2) (layer "B.Cu") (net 1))
 (segment (start 139.656377 102.277709) (end 139.679937 102.277709) (width 0.2) (layer "B.Cu") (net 1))
 (segment (start 139.679937 102.277709) (end 140.240839 101.716807) (width 0.2) (layer "B.Cu") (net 1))
 (segment (start 139.656377 94.777709) (end 139.656377 94.598887) (width 0.2) (layer "B.Cu") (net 1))
 (segment (start 140.316966 93.438298) (end 139.656377 92.777709) (width 0.2) (layer "B.Cu") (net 1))
 (segment (start 139.656377 95.098887) (end 139.316966 95.438298) (width 0.2) (layer "B.Cu") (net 1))
 (segment (start 135.648393 96.512365) (end 136.1928 97.056772) (width 0.2) (layer "F.Cu") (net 9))
 (segment (start 136.1928 97.056772) (end 136.1928 97.741286) (width 0.2) (layer "F.Cu") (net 9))
 (segment (start 136.1928 97.741286) (end 136.156377 97.777709) (width 0.2) (layer "F.Cu") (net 9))
 (via (at 136.156377 97.777709) (size 0.6) (drill 0.3) (layers "F.Cu" "B.Cu") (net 9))
 (segment (start 135.720481 97.005414) (end 135.720481 96.022582) (width 0.2) (layer "B.Cu") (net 9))
 (segment (start 136.156377 97.777709) (end 136.488387 97.777709) (width 0.2) (layer "B.Cu") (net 9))
 (segment (start 135.720481 96.022582) (end 131.855608 92.157709) (width 0.2) (layer "B.Cu") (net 9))
 (segment (start 136.156377 97.44131) (end 135.720481 97.005414) (width 0.2) (layer "B.Cu") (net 9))
 (segment (start 136.156377 97.777709) (end 136.156377 97.44131) (width 0.2) (layer "B.Cu") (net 9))
 (segment (start 136.488387 97.777709) (end 136.909784 98.199106) (width 0.2) (layer "B.Cu") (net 9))
 (segment (start 136.001946 96.158812) (end 136.620843 96.777709) (width 0.2) (layer "F.Cu") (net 8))
 (segment (start 136.620843 96.777709) (end 137.156377 96.777709) (width 0.2) (layer "F.Cu") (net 8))
 (via (at 137.156377 96.777709) (size 0.6) (drill 0.3) (layers "F.Cu" "B.Cu") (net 8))
 (segment (start 136.85042 96.777709) (end 136.399303 96.326592) (width 0.2) (layer "B.Cu") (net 8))
 (segment (start 136.399303 94.161404) (end 131.855608 89.617709) (width 0.2) (layer "B.Cu") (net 8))
 (segment (start 137.156377 96.777709) (end 136.85042 96.777709) (width 0.2) (layer "B.Cu") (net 8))
 (segment (start 137.156377 96.777709) (end 137.156377 97.088055) (width 0.2) (layer "B.Cu") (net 8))
 (segment (start 137.156377 97.088055) (end 137.588606 97.520284) (width 0.2) (layer "B.Cu") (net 8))
 (segment (start 136.399303 96.326592) (end 136.399303 94.161404) (width 0.2) (layer "B.Cu") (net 8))
 (segment (start 144.363484 99.570602) (end 144.863484 99.570602) (width 0.2) (layer "F.Cu") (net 34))
 (segment (start 144.863484 99.570602) (end 145.156377 99.277709) (width 0.2) (layer "F.Cu") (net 34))
 (via (at 145.156377 99.277709) (size 0.6) (drill 0.3) (layers "F.Cu" "B.Cu") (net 34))
 (segment (start 145.656377 99.777709) (end 147.095608 99.777709) (width 0.2) (layer "B.Cu") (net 34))
 (segment (start 145.156377 99.277709) (end 144.750444 99.277709) (width 0.2) (layer "B.Cu") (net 34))
 (segment (start 145.156377 99.277709) (end 145.656377 99.777709) (width 0.2) (layer "B.Cu") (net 34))
 (segment (start 144.750444 99.277709) (end 144.473858 99.554295) (width 0.2) (layer "B.Cu") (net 34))
 (segment (start 144.473858 99.554295) (end 143.432963 99.554295) (width 0.2) (layer "B.Cu") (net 34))
 (segment (start 135.256377 80.318478) (end 131.855608 76.917709) (width 0.2) (layer "F.Cu") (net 3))
 (segment (start 137.769713 94.391045) (end 135.256377 91.877709) (width 0.2) (layer "F.Cu") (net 3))
 (segment (start 135.256377 91.877709) (end 135.256377 80.318478) (width 0.2) (layer "F.Cu") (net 3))
 (segment (start 136.709053 101.691923) (end 135.656377 102.744599) (width 0.2) (layer "F.Cu") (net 19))
 (segment (start 135.656377 102.744599) (end 135.656377 113.75694) (width 0.2) (layer "F.Cu") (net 19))
 (segment (start 135.656377 113.75694) (end 131.855608 117.557709) (width 0.2) (layer "F.Cu") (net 19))
 (segment (start 137.416159 102.399029) (end 136.456377 103.358811) (width 0.2) (layer "F.Cu") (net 21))
 (segment (start 136.456377 103.358811) (end 136.456377 118.03694) (width 0.2) (layer "F.Cu") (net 21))
 (segment (start 136.456377 118.03694) (end 131.855608 122.637709) (width 0.2) (layer "F.Cu") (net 21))
 (segment (start 136.856377 103.665919) (end 136.856377 120.17694) (width 0.2) (layer "F.Cu") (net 22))
 (segment (start 136.856377 120.17694) (end 131.855608 125.177709) (width 0.2) (layer "F.Cu") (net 22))
 (segment (start 137.769713 102.752583) (end 136.856377 103.665919) (width 0.2) (layer "F.Cu") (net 22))
 (segment (start 134.056377 101.445461) (end 134.056377 105.19694) (width 0.2) (layer "F.Cu") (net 15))
 (segment (start 134.056377 105.19694) (end 131.855608 107.397709) (width 0.2) (layer "F.Cu") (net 15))
 (segment (start 135.224129 100.277709) (end 134.056377 101.445461) (width 0.2) (layer "F.Cu") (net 15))
 (segment (start 135.294839 100.277709) (end 135.224129 100.277709) (width 0.2) (layer "F.Cu") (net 15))
 (segment (start 134.941286 97.219472) (end 134.396879 96.675065) (width 0.2) (layer "F.Cu") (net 11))
 (segment (start 132.418252 96.675065) (end 131.855608 97.237709) (width 0.2) (layer "F.Cu") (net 11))
 (segment (start 134.396879 96.675065) (end 132.418252 96.675065) (width 0.2) (layer "F.Cu") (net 11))
 (segment (start 131.855608 104.857709) (end 133.656377 103.05694) (width 0.2) (layer "F.Cu") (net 14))
 (segment (start 133.656377 103.05694) (end 133.656377 101.209065) (width 0.2) (layer "F.Cu") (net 14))
 (segment (start 133.656377 101.209065) (end 134.941286 99.924156) (width 0.2) (layer "F.Cu") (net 14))
 (segment (start 136.001946 100.984816) (end 134.856377 102.130385) (width 0.2) (layer "F.Cu") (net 17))
 (segment (start 134.856377 109.47694) (end 131.855608 112.477709) (width 0.2) (layer "F.Cu") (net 17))
 (segment (start 134.856377 102.130385) (end 134.856377 109.47694) (width 0.2) (layer "F.Cu") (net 17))
 (segment (start 133.656377 88.878478) (end 133.656377 93.106137) (width 0.2) (layer "F.Cu") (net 7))
 (segment (start 133.656377 93.106137) (end 136.355499 95.805259) (width 0.2) (layer "F.Cu") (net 7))
 (segment (start 131.855608 87.077709) (end 133.656377 88.878478) (width 0.2) (layer "F.Cu") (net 7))
 (segment (start 136.355499 101.338369) (end 135.256377 102.437491) (width 0.2) (layer "F.Cu") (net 18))
 (segment (start 135.256377 102.437491) (end 135.256377 111.61694) (width 0.2) (layer "F.Cu") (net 18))
 (segment (start 135.256377 111.61694) (end 131.855608 115.017709) (width 0.2) (layer "F.Cu") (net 18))
 (segment (start 133.126629 94.697709) (end 131.855608 94.697709) (width 0.2) (layer "F.Cu") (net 10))
 (segment (start 135.294839 96.865919) (end 133.126629 94.697709) (width 0.2) (layer "F.Cu") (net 10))
 (segment (start 134.060291 97.573026) (end 131.855608 99.777709) (width 0.2) (layer "F.Cu") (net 12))
 (segment (start 134.587732 97.573026) (end 134.060291 97.573026) (width 0.2) (layer "F.Cu") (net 12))
 (segment (start 134.056377 86.738478) (end 131.855608 84.537709) (width 0.2) (layer "F.Cu") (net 6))
 (segment (start 136.709053 95.451705) (end 134.056377 92.799029) (width 0.2) (layer "F.Cu") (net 6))
 (segment (start 134.056377 92.799029) (end 134.056377 86.738478) (width 0.2) (layer "F.Cu") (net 6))
 (segment (start 134.587732 99.570602) (end 134.587732 99.585585) (width 0.2) (layer "F.Cu") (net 13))
 (segment (start 134.587732 99.585585) (end 131.855608 102.317709) (width 0.2) (layer "F.Cu") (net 13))
 (segment (start 134.456377 107.33694) (end 131.855608 109.937709) (width 0.2) (layer "F.Cu") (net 16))
 (segment (start 134.456377 101.823279) (end 134.456377 107.33694) (width 0.2) (layer "F.Cu") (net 16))
 (segment (start 135.648393 100.631263) (end 134.456377 101.823279) (width 0.2) (layer "F.Cu") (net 16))
 (segment (start 138.123266 94.037492) (end 135.656377 91.570603) (width 0.2) (layer "F.Cu") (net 2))
 (segment (start 135.656377 78.178478) (end 131.855608 74.377709) (width 0.2) (layer "F.Cu") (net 2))
 (segment (start 135.656377 91.570603) (end 135.656377 78.178478) (width 0.2) (layer "F.Cu") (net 2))
 (segment (start 134.456377 92.491923) (end 134.456377 84.598478) (width 0.2) (layer "F.Cu") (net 5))
 (segment (start 137.062606 95.098152) (end 134.456377 92.491923) (width 0.2) (layer "F.Cu") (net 5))
 (segment (start 134.456377 84.598478) (end 131.855608 81.997709) (width 0.2) (layer "F.Cu") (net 5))
 (segment (start 136.056377 115.89694) (end 131.855608 120.097709) (width 0.2) (layer "F.Cu") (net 20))
 (segment (start 137.062606 102.045476) (end 136.056377 103.051705) (width 0.2) (layer "F.Cu") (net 20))
 (segment (start 136.056377 103.051705) (end 136.056377 115.89694) (width 0.2) (layer "F.Cu") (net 20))
 (segment (start 137.416159 94.744599) (end 134.856377 92.184817) (width 0.2) (layer "F.Cu") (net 4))
 (segment (start 134.856377 92.184817) (end 134.856377 82.458478) (width 0.2) (layer "F.Cu") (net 4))
 (segment (start 134.856377 82.458478) (end 131.855608 79.457709) (width 0.2) (layer "F.Cu") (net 4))
 (segment (start 145.156377 103.191923) (end 142.94927 100.984816) (width 0.2) (layer "F.Cu") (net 31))
 (segment (start 147.095608 107.397709) (end 145.156377 105.458478) (width 0.2) (layer "F.Cu") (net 31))
 (segment (start 145.156377 105.458478) (end 145.156377 103.191923) (width 0.2) (layer "F.Cu") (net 31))
 (segment (start 143.956377 94.477709) (end 143.956377 87.67694) (width 0.2) (layer "F.Cu") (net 40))
 (segment (start 142.595717 95.805259) (end 142.628827 95.805259) (width 0.2) (layer "F.Cu") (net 40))
 (segment (start 142.628827 95.805259) (end 143.956377 94.477709) (width 0.2) (layer "F.Cu") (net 40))
 (segment (start 143.956377 87.67694) (end 147.095608 84.537709) (width 0.2) (layer "F.Cu") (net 40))
 (segment (start 144.356377 109.738478) (end 147.095608 112.477709) (width 0.2) (layer "F.Cu") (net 29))
 (segment (start 142.242163 101.691923) (end 144.356377 103.806137) (width 0.2) (layer "F.Cu") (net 29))
 (segment (start 144.356377 103.806137) (end 144.356377 109.738478) (width 0.2) (layer "F.Cu") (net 29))
 (segment (start 141.181503 94.391045) (end 142.356377 93.216171) (width 0.2) (layer "F.Cu") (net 44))
 (segment (start 142.356377 79.11694) (end 147.095608 74.377709) (width 0.2) (layer "F.Cu") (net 44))
 (segment (start 142.356377 93.216171) (end 142.356377 79.11694) (width 0.2) (layer "F.Cu") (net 44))
 (segment (start 144.00993 97.219472) (end 146.531693 94.697709) (width 0.2) (layer "F.Cu") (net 36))
 (segment (start 146.531693 94.697709) (end 147.095608 94.697709) (width 0.2) (layer "F.Cu") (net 36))
 (segment (start 142.242163 95.451705) (end 142.312875 95.451705) (width 0.2) (layer "F.Cu") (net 41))
 (segment (start 143.556377 85.53694) (end 147.095608 81.997709) (width 0.2) (layer "F.Cu") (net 41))
 (segment (start 143.556377 94.208203) (end 143.556377 85.53694) (width 0.2) (layer "F.Cu") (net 41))
 (segment (start 142.312875 95.451705) (end 143.556377 94.208203) (width 0.2) (layer "F.Cu") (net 41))
 (segment (start 142.356377 105.341671) (end 142.356377 120.438478) (width 0.2) (layer "F.Cu") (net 24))
 (segment (start 142.356377 120.438478) (end 147.095608 125.177709) (width 0.2) (layer "F.Cu") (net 24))
 (segment (start 140.474396 103.45969) (end 142.356377 105.341671) (width 0.2) (layer "F.Cu") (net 24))
 (segment (start 142.756377 118.298478) (end 147.095608 122.637709) (width 0.2) (layer "F.Cu") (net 25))
 (segment (start 142.756377 105.034563) (end 142.756377 118.298478) (width 0.2) (layer "F.Cu") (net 25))
 (segment (start 140.82795 103.106136) (end 142.756377 105.034563) (width 0.2) (layer "F.Cu") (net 25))
 (segment (start 143.956377 104.113243) (end 143.956377 111.878478) (width 0.2) (layer "F.Cu") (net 28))
 (segment (start 143.956377 111.878478) (end 147.095608 115.017709) (width 0.2) (layer "F.Cu") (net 28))
 (segment (start 141.88861 102.045476) (end 143.956377 104.113243) (width 0.2) (layer "F.Cu") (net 28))
 (segment (start 144.756377 95.058811) (end 144.756377 91.95694) (width 0.2) (layer "F.Cu") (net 38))
 (segment (start 144.756377 91.95694) (end 147.095608 89.617709) (width 0.2) (layer "F.Cu") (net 38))
 (segment (start 143.302823 96.512365) (end 144.756377 95.058811) (width 0.2) (layer "F.Cu") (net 38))
 (segment (start 145.156377 95.365919) (end 143.656377 96.865919) (width 0.2) (layer "F.Cu") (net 37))
 (segment (start 145.156377 94.09694) (end 145.156377 95.365919) (width 0.2) (layer "F.Cu") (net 37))
 (segment (start 147.095608 92.157709) (end 145.156377 94.09694) (width 0.2) (layer "F.Cu") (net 37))
 (segment (start 143.302823 100.631263) (end 147.095608 104.424048) (width 0.2) (layer "F.Cu") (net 32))
 (segment (start 147.095608 104.424048) (end 147.095608 104.857709) (width 0.2) (layer "F.Cu") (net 32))
 (segment (start 141.88861 95.098152) (end 143.156377 93.830385) (width 0.2) (layer "F.Cu") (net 42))
 (segment (start 143.156377 83.39694) (end 147.095608 79.457709) (width 0.2) (layer "F.Cu") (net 42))
 (segment (start 143.156377 93.830385) (end 143.156377 83.39694) (width 0.2) (layer "F.Cu") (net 42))
 (segment (start 142.756377 81.25694) (end 147.095608 76.917709) (width 0.2) (layer "F.Cu") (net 43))
 (segment (start 142.756377 93.523279) (end 142.756377 81.25694) (width 0.2) (layer "F.Cu") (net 43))
 (segment (start 141.535057 94.744599) (end 142.756377 93.523279) (width 0.2) (layer "F.Cu") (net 43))
 (segment (start 144.363484 97.573026) (end 146.760291 97.573026) (width 0.2) (layer "F.Cu") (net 35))
 (segment (start 146.760291 97.573026) (end 147.095608 97.237709) (width 0.2) (layer "F.Cu") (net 35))
 (segment (start 144.356377 89.81694) (end 147.095608 87.077709) (width 0.2) (layer "F.Cu") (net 39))
 (segment (start 142.94927 96.158812) (end 144.356377 94.751705) (width 0.2) (layer "F.Cu") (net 39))
 (segment (start 144.356377 94.751705) (end 144.356377 89.81694) (width 0.2) (layer "F.Cu") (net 39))
 (segment (start 144.756377 103.499029) (end 144.756377 107.598478) (width 0.2) (layer "F.Cu") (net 30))
 (segment (start 142.595717 101.338369) (end 144.756377 103.499029) (width 0.2) (layer "F.Cu") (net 30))
 (segment (start 144.756377 107.598478) (end 147.095608 109.937709) (width 0.2) (layer "F.Cu") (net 30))
 (segment (start 143.656377 100.277709) (end 145.696377 102.317709) (width 0.2) (layer "F.Cu") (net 33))
 (segment (start 145.696377 102.317709) (end 147.095608 102.317709) (width 0.2) (layer "F.Cu") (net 33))
 (segment (start 143.556377 114.018478) (end 147.095608 117.557709) (width 0.2) (layer "F.Cu") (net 27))
 (segment (start 143.556377 104.349639) (end 143.556377 114.018478) (width 0.2) (layer "F.Cu") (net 27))
 (segment (start 141.605767 102.399029) (end 143.556377 104.349639) (width 0.2) (layer "F.Cu") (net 27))
 (segment (start 141.535057 102.399029) (end 141.605767 102.399029) (width 0.2) (layer "F.Cu") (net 27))
 (segment (start 143.156377 104.727457) (end 143.156377 116.158478) (width 0.2) (layer "F.Cu") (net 26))
 (segment (start 143.156377 116.158478) (end 147.095608 120.097709) (width 0.2) (layer "F.Cu") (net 26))
 (segment (start 141.181503 102.752583) (end 143.156377 104.727457) (width 0.2) (layer "F.Cu") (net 26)))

